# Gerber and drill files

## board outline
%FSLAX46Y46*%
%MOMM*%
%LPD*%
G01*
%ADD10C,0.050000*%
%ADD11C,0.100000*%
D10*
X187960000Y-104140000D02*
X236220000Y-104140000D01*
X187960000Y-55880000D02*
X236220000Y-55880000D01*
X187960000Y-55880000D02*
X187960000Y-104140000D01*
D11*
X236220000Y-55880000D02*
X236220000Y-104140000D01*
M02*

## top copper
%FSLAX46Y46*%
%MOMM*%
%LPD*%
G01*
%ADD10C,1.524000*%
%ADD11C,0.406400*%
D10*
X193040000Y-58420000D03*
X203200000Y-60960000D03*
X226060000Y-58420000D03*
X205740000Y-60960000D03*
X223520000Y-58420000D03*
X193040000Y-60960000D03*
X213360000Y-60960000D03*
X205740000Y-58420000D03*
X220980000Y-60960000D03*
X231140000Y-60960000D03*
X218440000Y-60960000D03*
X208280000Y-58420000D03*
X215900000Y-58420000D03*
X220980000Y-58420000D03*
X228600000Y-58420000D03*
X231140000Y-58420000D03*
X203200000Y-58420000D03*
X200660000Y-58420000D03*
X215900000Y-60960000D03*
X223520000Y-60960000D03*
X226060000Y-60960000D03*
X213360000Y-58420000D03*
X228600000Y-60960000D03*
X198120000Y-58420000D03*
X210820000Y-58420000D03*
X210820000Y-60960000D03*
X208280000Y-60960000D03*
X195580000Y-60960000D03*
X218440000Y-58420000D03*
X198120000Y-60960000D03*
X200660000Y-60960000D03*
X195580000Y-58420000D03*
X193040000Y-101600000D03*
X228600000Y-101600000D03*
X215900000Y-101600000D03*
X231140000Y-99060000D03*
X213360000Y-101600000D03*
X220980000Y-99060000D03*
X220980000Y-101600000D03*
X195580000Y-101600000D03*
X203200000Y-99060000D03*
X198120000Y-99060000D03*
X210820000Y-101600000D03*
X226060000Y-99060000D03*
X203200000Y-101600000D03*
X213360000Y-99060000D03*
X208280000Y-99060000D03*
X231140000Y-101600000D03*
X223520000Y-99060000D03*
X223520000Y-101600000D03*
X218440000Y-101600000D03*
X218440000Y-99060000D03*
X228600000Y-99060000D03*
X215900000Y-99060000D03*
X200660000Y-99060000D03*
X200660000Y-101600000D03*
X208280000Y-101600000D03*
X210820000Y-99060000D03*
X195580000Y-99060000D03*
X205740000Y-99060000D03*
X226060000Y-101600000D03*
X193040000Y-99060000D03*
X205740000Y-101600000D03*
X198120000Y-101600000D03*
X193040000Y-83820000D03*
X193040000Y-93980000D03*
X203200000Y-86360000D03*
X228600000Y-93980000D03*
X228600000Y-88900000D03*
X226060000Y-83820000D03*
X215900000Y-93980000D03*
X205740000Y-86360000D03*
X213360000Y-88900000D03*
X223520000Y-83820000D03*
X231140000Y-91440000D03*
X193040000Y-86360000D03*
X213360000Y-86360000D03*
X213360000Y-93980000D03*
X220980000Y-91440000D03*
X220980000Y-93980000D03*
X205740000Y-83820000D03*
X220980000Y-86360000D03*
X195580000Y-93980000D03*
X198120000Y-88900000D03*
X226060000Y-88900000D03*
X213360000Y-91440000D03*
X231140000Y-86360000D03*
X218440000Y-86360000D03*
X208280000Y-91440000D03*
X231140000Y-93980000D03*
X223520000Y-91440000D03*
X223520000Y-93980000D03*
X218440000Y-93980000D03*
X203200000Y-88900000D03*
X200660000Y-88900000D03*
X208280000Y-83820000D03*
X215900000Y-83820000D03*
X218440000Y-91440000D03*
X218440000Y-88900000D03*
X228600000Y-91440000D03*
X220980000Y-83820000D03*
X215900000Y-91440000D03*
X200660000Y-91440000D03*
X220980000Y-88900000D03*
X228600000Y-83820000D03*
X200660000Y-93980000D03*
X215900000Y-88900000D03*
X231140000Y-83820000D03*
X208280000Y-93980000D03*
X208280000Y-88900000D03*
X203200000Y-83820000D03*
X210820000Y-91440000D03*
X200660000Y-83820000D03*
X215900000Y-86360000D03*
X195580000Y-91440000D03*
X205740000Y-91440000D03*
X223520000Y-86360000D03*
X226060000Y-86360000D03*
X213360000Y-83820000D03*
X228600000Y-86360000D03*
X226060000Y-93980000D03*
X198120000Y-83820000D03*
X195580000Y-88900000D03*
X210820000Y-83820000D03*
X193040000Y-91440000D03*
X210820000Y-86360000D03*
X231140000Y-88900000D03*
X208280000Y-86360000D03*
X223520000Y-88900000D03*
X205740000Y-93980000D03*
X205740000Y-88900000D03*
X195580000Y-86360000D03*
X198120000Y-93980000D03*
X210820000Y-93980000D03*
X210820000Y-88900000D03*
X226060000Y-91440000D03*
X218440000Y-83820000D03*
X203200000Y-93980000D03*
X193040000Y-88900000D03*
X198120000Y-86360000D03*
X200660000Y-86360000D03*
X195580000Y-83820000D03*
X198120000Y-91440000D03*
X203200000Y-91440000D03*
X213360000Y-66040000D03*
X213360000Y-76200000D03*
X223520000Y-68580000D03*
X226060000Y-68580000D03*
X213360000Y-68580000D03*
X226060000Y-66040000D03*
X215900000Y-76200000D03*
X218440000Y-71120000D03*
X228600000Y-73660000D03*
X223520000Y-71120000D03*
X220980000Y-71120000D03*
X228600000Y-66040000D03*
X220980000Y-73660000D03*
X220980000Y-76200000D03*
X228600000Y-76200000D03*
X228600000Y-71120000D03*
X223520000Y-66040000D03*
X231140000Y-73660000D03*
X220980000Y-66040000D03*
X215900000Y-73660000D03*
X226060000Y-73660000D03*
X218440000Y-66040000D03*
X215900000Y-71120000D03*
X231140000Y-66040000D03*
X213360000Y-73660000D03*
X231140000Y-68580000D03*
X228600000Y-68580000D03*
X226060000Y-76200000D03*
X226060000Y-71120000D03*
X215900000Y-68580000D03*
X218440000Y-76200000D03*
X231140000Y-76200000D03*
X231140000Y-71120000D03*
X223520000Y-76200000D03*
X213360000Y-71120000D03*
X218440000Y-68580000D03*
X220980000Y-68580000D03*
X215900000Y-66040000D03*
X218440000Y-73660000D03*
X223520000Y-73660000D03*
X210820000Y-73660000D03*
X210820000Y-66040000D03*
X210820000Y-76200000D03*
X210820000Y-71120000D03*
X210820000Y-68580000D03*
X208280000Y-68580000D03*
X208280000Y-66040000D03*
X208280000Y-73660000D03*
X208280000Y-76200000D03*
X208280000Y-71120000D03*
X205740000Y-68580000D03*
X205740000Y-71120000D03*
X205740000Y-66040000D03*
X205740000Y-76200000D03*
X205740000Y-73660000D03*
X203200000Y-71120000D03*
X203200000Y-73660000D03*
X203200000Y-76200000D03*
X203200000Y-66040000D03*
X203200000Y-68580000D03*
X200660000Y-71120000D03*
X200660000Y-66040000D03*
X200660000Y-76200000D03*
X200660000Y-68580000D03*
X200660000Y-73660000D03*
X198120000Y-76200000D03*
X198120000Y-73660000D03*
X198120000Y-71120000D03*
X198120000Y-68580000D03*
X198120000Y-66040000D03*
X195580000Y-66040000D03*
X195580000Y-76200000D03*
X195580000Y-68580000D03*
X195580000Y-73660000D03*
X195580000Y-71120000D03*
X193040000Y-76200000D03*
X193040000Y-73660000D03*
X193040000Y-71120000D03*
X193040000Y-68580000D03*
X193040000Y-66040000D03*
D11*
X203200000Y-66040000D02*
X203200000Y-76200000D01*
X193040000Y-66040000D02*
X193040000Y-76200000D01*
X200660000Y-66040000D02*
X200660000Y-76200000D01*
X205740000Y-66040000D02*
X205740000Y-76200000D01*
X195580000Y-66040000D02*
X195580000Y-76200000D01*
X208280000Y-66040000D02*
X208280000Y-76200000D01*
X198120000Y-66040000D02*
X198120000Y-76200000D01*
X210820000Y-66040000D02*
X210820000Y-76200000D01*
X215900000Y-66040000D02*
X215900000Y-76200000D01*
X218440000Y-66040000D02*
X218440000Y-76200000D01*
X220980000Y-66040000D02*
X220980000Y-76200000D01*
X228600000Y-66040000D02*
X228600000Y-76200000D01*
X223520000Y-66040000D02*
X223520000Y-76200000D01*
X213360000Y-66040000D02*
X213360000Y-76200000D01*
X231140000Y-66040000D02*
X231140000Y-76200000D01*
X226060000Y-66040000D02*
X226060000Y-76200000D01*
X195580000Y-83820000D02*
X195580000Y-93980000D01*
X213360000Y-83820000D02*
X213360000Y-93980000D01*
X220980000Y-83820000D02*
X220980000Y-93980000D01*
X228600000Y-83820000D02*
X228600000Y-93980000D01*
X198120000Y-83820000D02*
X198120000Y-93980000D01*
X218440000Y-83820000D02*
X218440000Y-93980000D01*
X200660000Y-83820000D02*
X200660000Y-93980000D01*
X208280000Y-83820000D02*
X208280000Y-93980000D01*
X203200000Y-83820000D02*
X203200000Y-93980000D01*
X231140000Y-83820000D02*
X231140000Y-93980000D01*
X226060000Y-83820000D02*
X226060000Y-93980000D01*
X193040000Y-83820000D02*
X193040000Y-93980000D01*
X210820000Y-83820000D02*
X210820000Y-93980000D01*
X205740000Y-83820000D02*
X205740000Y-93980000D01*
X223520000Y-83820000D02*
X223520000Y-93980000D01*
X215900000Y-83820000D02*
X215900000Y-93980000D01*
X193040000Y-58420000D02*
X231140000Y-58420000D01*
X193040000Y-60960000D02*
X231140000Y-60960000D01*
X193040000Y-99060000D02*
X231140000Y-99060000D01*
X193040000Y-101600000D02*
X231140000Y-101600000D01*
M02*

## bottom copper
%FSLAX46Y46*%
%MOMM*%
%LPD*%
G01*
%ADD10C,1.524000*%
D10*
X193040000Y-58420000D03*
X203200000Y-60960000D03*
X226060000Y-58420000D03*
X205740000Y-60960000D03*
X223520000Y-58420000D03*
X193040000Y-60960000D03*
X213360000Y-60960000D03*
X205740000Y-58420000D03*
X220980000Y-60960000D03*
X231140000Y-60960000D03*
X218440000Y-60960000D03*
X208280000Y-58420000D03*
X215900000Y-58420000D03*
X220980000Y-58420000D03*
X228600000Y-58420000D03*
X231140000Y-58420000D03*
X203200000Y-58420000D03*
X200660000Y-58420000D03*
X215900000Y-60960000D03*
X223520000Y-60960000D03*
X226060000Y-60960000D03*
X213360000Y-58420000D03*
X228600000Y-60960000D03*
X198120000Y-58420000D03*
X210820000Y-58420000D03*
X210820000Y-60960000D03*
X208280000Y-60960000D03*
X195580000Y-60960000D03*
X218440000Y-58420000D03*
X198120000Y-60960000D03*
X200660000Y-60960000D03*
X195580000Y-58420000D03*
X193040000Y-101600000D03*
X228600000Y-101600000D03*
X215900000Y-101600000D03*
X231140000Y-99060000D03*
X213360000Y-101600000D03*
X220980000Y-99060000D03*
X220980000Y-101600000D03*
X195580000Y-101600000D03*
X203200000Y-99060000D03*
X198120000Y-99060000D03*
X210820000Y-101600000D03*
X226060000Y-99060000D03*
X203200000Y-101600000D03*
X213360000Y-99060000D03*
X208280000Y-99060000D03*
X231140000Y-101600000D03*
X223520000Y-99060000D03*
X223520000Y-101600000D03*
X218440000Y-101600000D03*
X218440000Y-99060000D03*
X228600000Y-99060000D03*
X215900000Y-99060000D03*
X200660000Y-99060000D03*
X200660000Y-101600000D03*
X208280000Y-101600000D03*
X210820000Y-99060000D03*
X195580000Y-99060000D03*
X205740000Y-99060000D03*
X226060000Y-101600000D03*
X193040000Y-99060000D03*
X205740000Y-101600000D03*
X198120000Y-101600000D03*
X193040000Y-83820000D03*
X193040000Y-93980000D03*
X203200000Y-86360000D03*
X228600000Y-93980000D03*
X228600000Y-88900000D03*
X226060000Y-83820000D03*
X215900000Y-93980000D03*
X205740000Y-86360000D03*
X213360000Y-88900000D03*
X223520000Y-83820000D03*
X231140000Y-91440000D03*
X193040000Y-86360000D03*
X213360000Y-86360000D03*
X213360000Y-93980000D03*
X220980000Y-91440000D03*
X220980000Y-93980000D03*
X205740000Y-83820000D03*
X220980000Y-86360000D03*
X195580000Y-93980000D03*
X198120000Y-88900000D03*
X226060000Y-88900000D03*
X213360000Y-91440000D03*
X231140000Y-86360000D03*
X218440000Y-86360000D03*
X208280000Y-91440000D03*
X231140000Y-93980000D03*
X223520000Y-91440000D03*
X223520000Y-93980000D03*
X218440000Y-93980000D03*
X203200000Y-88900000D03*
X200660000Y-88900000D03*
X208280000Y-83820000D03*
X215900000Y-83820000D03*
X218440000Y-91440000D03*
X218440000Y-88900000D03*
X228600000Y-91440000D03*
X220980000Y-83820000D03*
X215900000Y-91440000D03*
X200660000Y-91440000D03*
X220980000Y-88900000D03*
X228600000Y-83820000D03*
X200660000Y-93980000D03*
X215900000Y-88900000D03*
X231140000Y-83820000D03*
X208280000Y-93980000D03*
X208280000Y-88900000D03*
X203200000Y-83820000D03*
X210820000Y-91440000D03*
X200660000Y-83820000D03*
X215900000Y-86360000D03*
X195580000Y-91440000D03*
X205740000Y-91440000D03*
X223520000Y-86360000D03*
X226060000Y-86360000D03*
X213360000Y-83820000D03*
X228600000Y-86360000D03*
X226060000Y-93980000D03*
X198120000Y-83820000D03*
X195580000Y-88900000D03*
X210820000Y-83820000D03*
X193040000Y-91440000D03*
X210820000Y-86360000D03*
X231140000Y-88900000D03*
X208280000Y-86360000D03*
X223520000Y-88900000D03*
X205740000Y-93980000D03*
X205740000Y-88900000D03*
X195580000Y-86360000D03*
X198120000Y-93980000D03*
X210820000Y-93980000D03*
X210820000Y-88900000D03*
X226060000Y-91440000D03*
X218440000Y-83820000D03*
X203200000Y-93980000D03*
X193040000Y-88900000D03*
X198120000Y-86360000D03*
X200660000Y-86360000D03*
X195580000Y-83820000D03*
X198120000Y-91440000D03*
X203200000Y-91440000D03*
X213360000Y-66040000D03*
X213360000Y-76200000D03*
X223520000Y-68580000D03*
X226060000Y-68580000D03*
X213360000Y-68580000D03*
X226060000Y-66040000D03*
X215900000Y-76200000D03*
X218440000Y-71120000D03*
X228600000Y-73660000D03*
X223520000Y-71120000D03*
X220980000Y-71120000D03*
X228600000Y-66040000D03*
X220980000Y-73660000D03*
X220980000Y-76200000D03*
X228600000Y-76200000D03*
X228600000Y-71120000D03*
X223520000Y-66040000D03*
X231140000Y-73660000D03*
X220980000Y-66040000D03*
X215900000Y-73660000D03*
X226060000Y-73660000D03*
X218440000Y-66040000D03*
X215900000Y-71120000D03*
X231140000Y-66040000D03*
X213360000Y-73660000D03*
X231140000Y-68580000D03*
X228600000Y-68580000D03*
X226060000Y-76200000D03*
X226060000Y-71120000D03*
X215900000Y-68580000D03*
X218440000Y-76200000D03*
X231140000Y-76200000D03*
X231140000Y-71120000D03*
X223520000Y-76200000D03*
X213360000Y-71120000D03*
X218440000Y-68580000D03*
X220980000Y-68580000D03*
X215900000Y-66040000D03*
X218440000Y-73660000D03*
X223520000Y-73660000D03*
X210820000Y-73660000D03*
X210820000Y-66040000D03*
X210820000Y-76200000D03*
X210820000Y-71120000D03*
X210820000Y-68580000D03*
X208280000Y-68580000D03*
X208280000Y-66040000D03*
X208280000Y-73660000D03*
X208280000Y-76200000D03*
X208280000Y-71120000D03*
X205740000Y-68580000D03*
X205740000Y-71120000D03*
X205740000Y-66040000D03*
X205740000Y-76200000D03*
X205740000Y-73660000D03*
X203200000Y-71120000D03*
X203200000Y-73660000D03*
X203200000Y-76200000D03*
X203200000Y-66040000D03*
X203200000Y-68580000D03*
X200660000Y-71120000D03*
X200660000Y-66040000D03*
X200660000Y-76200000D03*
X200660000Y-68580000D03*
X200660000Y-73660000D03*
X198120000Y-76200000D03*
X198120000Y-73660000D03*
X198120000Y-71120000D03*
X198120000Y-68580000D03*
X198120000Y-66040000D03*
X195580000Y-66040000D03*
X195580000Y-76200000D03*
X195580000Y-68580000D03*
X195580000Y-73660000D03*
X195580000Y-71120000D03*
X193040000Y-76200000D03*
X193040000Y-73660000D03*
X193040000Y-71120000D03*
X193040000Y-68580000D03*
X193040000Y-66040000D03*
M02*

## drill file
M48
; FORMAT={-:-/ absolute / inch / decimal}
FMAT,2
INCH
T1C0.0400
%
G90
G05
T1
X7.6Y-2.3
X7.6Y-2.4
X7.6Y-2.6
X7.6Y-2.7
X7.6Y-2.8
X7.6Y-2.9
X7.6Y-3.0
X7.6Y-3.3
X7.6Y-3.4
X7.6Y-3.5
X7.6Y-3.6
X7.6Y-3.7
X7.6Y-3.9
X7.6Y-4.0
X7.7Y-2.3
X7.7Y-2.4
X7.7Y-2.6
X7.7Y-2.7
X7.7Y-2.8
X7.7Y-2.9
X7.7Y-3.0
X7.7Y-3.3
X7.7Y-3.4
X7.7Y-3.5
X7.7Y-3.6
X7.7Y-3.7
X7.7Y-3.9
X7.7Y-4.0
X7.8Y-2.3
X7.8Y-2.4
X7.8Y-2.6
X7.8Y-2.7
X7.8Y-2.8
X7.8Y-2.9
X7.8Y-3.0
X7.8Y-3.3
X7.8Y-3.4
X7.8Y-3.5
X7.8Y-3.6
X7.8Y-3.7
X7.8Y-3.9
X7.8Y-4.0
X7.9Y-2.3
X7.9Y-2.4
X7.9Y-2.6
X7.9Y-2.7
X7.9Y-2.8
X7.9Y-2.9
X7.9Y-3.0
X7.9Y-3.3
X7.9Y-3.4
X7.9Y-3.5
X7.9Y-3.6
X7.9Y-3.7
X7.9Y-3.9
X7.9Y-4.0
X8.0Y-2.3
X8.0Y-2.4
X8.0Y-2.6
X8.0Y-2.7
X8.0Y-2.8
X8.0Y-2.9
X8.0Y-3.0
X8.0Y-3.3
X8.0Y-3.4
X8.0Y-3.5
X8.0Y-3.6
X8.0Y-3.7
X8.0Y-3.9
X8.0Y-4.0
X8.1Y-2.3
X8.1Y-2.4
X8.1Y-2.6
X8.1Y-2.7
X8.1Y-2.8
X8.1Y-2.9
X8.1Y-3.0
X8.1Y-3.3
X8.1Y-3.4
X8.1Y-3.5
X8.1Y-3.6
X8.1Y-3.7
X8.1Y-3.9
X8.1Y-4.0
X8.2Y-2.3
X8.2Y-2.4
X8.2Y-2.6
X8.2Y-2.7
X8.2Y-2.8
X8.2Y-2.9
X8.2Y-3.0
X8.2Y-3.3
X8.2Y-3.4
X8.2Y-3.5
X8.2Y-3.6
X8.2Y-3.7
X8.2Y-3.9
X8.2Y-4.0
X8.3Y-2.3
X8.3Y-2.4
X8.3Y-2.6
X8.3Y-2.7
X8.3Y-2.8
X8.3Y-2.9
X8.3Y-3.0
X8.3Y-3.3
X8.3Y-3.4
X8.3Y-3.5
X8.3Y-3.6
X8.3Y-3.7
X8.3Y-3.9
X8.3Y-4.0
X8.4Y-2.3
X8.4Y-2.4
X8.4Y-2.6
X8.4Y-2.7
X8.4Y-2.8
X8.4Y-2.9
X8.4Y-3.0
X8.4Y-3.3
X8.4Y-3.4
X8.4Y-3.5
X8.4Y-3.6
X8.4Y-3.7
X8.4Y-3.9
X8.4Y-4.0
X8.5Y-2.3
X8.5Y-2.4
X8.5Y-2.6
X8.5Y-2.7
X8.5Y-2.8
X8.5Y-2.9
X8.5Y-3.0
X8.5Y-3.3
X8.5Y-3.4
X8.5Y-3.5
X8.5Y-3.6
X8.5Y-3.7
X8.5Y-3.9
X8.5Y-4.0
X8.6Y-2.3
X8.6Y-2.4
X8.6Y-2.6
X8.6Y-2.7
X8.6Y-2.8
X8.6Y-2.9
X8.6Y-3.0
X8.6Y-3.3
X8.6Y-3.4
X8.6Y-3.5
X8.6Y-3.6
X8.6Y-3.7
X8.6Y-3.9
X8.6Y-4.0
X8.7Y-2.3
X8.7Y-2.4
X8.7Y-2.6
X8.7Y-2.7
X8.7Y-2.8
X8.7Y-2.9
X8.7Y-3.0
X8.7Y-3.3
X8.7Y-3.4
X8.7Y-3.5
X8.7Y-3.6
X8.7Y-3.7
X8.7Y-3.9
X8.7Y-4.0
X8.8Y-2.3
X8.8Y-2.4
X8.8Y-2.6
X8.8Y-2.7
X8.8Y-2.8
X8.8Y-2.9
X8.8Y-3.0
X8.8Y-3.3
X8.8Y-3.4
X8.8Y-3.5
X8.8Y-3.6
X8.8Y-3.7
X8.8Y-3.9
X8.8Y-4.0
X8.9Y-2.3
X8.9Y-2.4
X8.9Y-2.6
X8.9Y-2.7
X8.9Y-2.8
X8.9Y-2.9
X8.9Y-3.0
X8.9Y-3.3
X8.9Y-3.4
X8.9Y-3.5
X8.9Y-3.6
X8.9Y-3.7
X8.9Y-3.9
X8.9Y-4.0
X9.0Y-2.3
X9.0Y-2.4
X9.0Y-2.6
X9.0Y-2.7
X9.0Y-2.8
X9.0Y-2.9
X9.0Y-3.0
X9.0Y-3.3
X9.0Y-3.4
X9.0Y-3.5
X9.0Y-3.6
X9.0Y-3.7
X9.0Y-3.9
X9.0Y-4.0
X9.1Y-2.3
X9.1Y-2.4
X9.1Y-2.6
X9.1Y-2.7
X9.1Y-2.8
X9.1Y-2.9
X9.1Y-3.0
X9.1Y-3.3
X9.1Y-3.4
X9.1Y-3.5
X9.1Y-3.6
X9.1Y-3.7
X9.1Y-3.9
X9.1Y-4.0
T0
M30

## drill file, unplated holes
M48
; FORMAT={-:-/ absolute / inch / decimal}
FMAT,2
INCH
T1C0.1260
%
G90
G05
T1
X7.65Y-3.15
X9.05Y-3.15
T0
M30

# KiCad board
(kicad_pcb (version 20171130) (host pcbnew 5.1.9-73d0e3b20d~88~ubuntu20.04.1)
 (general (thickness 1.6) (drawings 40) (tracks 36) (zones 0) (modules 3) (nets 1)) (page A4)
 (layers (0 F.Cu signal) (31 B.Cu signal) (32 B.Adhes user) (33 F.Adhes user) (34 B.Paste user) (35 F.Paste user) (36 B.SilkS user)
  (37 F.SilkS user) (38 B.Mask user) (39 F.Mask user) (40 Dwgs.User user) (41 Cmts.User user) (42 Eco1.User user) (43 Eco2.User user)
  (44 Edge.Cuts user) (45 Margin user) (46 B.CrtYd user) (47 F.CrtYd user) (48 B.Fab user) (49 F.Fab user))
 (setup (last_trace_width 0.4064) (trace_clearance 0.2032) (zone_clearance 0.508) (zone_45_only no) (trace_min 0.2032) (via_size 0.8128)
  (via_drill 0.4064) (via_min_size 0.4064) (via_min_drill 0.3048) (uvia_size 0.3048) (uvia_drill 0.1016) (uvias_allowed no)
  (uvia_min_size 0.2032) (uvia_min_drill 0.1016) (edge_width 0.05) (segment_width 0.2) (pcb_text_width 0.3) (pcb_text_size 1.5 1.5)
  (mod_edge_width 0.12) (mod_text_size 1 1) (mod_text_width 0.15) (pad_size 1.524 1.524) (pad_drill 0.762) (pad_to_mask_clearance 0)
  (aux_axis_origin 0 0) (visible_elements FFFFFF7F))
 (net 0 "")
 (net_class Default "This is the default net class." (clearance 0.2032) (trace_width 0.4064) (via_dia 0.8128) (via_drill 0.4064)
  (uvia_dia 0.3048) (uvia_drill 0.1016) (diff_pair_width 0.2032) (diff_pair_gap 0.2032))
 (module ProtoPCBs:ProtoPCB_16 (layer F.Cu) (at 193.04 58.42)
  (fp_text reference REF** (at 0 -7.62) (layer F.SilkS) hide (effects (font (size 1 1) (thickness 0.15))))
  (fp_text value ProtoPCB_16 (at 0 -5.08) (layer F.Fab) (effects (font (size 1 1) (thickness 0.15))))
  (pad 1 thru_hole circle (at 0 0) (size 1.524 1.524) (drill 1.016) (layers *.Cu *.Mask))
  (pad 1 thru_hole circle (at 10.16 2.54) (size 1.524 1.524) (drill 1.016) (layers *.Cu *.Mask))
  (pad 1 thru_hole circle (at 33.02 0) (size 1.524 1.524) (drill 1.016) (layers *.Cu *.Mask))
  (pad 1 thru_hole circle (at 12.7 2.54) (size 1.524 1.524) (drill 1.016) (layers *.Cu *.Mask))
  (pad 1 thru_hole circle (at 30.48 0) (size 1.524 1.524) (drill 1.016) (layers *.Cu *.Mask))
  (pad 1 thru_hole circle (at 0 2.54) (size 1.524 1.524) (drill 1.016) (layers *.Cu *.Mask))
  (pad 1 thru_hole circle (at 20.32 2.54) (size 1.524 1.524) (drill 1.016) (layers *.Cu *.Mask))
  (pad 1 thru_hole circle (at 12.7 0) (size 1.524 1.524) (drill 1.016) (layers *.Cu *.Mask))
  (pad 1 thru_hole circle (at 27.94 2.54) (size 1.524 1.524) (drill 1.016) (layers *.Cu *.Mask))
  (pad 1 thru_hole circle (at 38.1 2.54) (size 1.524 1.524) (drill 1.016) (layers *.Cu *.Mask))
  (pad 1 thru_hole circle (at 25.4 2.54) (size 1.524 1.524) (drill 1.016) (layers *.Cu *.Mask))
  (pad 1 thru_hole circle (at 15.24 0) (size 1.524 1.524) (drill 1.016) (layers *.Cu *.Mask))
  (pad 1 thru_hole circle (at 22.86 0) (size 1.524 1.524) (drill 1.016) (layers *.Cu *.Mask))
  (pad 1 thru_hole circle (at 27.94 0) (size 1.524 1.524) (drill 1.016) (layers *.Cu *.Mask))
  (pad 1 thru_hole circle (at 35.56 0) (size 1.524 1.524) (drill 1.016) (layers *.Cu *.Mask))
  (pad 1 thru_hole circle (at 38.1 0) (size 1.524 1.524) (drill 1.016) (layers *.Cu *.Mask))
  (pad 1 thru_hole circle (at 10.16 0) (size 1.524 1.524) (drill 1.016) (layers *.Cu *.Mask))
  (pad 1 thru_hole circle (at 7.62 0) (size 1.524 1.524) (drill 1.016) (layers *.Cu *.Mask))
  (pad 1 thru_hole circle (at 22.86 2.54) (size 1.524 1.524) (drill 1.016) (layers *.Cu *.Mask))
  (pad 1 thru_hole circle (at 30.48 2.54) (size 1.524 1.524) (drill 1.016) (layers *.Cu *.Mask))
  (pad 1 thru_hole circle (at 33.02 2.54) (size 1.524 1.524) (drill 1.016) (layers *.Cu *.Mask))
  (pad 1 thru_hole circle (at 20.32 0) (size 1.524 1.524) (drill 1.016) (layers *.Cu *.Mask))
  (pad 1 thru_hole circle (at 35.56 2.54) (size 1.524 1.524) (drill 1.016) (layers *.Cu *.Mask))
  (pad 1 thru_hole circle (at 5.08 0) (size 1.524 1.524) (drill 1.016) (layers *.Cu *.Mask))
  (pad 1 thru_hole circle (at 17.78 0) (size 1.524 1.524) (drill 1.016) (layers *.Cu *.Mask))
  (pad 1 thru_hole circle (at 17.78 2.54) (size 1.524 1.524) (drill 1.016) (layers *.Cu *.Mask))
  (pad 1 thru_hole circle (at 15.24 2.54) (size 1.524 1.524) (drill 1.016) (layers *.Cu *.Mask))
  (pad 1 thru_hole circle (at 2.54 2.54) (size 1.524 1.524) (drill 1.016) (layers *.Cu *.Mask))
  (pad 1 thru_hole circle (at 25.4 0) (size 1.524 1.524) (drill 1.016) (layers *.Cu *.Mask))
  (pad 1 thru_hole circle (at 5.08 2.54) (size 1.524 1.524) (drill 1.016) (layers *.Cu *.Mask))
  (pad 1 thru_hole circle (at 7.62 2.54) (size 1.524 1.524) (drill 1.016) (layers *.Cu *.Mask))
  (pad 1 thru_hole circle (at 2.54 0) (size 1.524 1.524) (drill 1.016) (layers *.Cu *.Mask))
  (pad 1 thru_hole circle (at 0 43.18) (size 1.524 1.524) (drill 1.016) (layers *.Cu *.Mask))
  (pad 1 thru_hole circle (at 35.56 43.18) (size 1.524 1.524) (drill 1.016) (layers *.Cu *.Mask))
  (pad 1 thru_hole circle (at 22.86 43.18) (size 1.524 1.524) (drill 1.016) (layers *.Cu *.Mask))
  (pad 1 thru_hole circle (at 38.1 40.64) (size 1.524 1.524) (drill 1.016) (layers *.Cu *.Mask))
  (pad 1 thru_hole circle (at 20.32 43.18) (size 1.524 1.524) (drill 1.016) (layers *.Cu *.Mask))
  (pad 1 thru_hole circle (at 27.94 40.64) (size 1.524 1.524) (drill 1.016) (layers *.Cu *.Mask))
  (pad 1 thru_hole circle (at 27.94 43.18) (size 1.524 1.524) (drill 1.016) (layers *.Cu *.Mask))
  (pad 1 thru_hole circle (at 2.54 43.18) (size 1.524 1.524) (drill 1.016) (layers *.Cu *.Mask))
  (pad 1 thru_hole circle (at 10.16 40.64) (size 1.524 1.524) (drill 1.016) (layers *.Cu *.Mask))
  (pad 1 thru_hole circle (at 5.08 40.64) (size 1.524 1.524) (drill 1.016) (layers *.Cu *.Mask))
  (pad 1 thru_hole circle (at 17.78 43.18) (size 1.524 1.524) (drill 1.016) (layers *.Cu *.Mask))
  (pad 1 thru_hole circle (at 33.02 40.64) (size 1.524 1.524) (drill 1.016) (layers *.Cu *.Mask))
  (pad 1 thru_hole circle (at 10.16 43.18) (size 1.524 1.524) (drill 1.016) (layers *.Cu *.Mask))
  (pad 1 thru_hole circle (at 20.32 40.64) (size 1.524 1.524) (drill 1.016) (layers *.Cu *.Mask))
  (pad 1 thru_hole circle (at 15.24 40.64) (size 1.524 1.524) (drill 1.016) (layers *.Cu *.Mask))
  (pad 1 thru_hole circle (at 38.1 43.18) (size 1.524 1.524) (drill 1.016) (layers *.Cu *.Mask))
  (pad 1 thru_hole circle (at 30.48 40.64) (size 1.524 1.524) (drill 1.016) (layers *.Cu *.Mask))
  (pad 1 thru_hole circle (at 30.48 43.18) (size 1.524 1.524) (drill 1.016) (layers *.Cu *.Mask))
  (pad 1 thru_hole circle (at 25.4 43.18) (size 1.524 1.524) (drill 1.016) (layers *.Cu *.Mask))
  (pad 1 thru_hole circle (at 25.4 40.64) (size 1.524 1.524) (drill 1.016) (layers *.Cu *.Mask))
  (pad 1 thru_hole circle (at 35.56 40.64) (size 1.524 1.524) (drill 1.016) (layers *.Cu *.Mask))
  (pad 1 thru_hole circle (at 22.86 40.64) (size 1.524 1.524) (drill 1.016) (layers *.Cu *.Mask))
  (pad 1 thru_hole circle (at 7.62 40.64) (size 1.524 1.524) (drill 1.016) (layers *.Cu *.Mask))
  (pad 1 thru_hole circle (at 7.62 43.18) (size 1.524 1.524) (drill 1.016) (layers *.Cu *.Mask))
  (pad 1 thru_hole circle (at 15.24 43.18) (size 1.524 1.524) (drill 1.016) (layers *.Cu *.Mask))
  (pad 1 thru_hole circle (at 17.78 40.64) (size 1.524 1.524) (drill 1.016) (layers *.Cu *.Mask))
  (pad 1 thru_hole circle (at 2.54 40.64) (size 1.524 1.524) (drill 1.016) (layers *.Cu *.Mask))
  (pad 1 thru_hole circle (at 12.7 40.64) (size 1.524 1.524) (drill 1.016) (layers *.Cu *.Mask))
  (pad 1 thru_hole circle (at 33.02 43.18) (size 1.524 1.524) (drill 1.016) (layers *.Cu *.Mask))
  (pad 1 thru_hole circle (at 0 40.64) (size 1.524 1.524) (drill 1.016) (layers *.Cu *.Mask))
  (pad 1 thru_hole circle (at 12.7 43.18) (size 1.524 1.524) (drill 1.016) (layers *.Cu *.Mask))
  (pad 1 thru_hole circle (at 5.08 43.18) (size 1.524 1.524) (drill 1.016) (layers *.Cu *.Mask))
  (pad 1 thru_hole circle (at 0 25.4) (size 1.524 1.524) (drill 1.016) (layers *.Cu *.Mask))
  (pad 1 thru_hole circle (at 0 35.56) (size 1.524 1.524) (drill 1.016) (layers *.Cu *.Mask))
  (pad 1 thru_hole circle (at 10.16 27.94) (size 1.524 1.524) (drill 1.016) (layers *.Cu *.Mask))
  (pad 1 thru_hole circle (at 35.56 35.56) (size 1.524 1.524) (drill 1.016) (layers *.Cu *.Mask))
  (pad 1 thru_hole circle (at 35.56 30.48) (size 1.524 1.524) (drill 1.016) (layers *.Cu *.Mask))
  (pad 1 thru_hole circle (at 33.02 25.4) (size 1.524 1.524) (drill 1.016) (layers *.Cu *.Mask))
  (pad 1 thru_hole circle (at 22.86 35.56) (size 1.524 1.524) (drill 1.016) (layers *.Cu *.Mask))
  (pad 1 thru_hole circle (at 12.7 27.94) (size 1.524 1.524) (drill 1.016) (layers *.Cu *.Mask))
  (pad 1 thru_hole circle (at 20.32 30.48) (size 1.524 1.524) (drill 1.016) (layers *.Cu *.Mask))
  (pad 1 thru_hole circle (at 30.48 25.4) (size 1.524 1.524) (drill 1.016) (layers *.Cu *.Mask))
  (pad 1 thru_hole circle (at 38.1 33.02) (size 1.524 1.524) (drill 1.016) (layers *.Cu *.Mask))
  (pad 1 thru_hole circle (at 0 27.94) (size 1.524 1.524) (drill 1.016) (layers *.Cu *.Mask))
  (pad 1 thru_hole circle (at 20.32 27.94) (size 1.524 1.524) (drill 1.016) (layers *.Cu *.Mask))
  (pad 1 thru_hole circle (at 20.32 35.56) (size 1.524 1.524) (drill 1.016) (layers *.Cu *.Mask))
  (pad 1 thru_hole circle (at 27.94 33.02) (size 1.524 1.524) (drill 1.016) (layers *.Cu *.Mask))
  (pad 1 thru_hole circle (at 27.94 35.56) (size 1.524 1.524) (drill 1.016) (layers *.Cu *.Mask))
  (pad 1 thru_hole circle (at 12.7 25.4) (size 1.524 1.524) (drill 1.016) (layers *.Cu *.Mask))
  (pad 1 thru_hole circle (at 27.94 27.94) (size 1.524 1.524) (drill 1.016) (layers *.Cu *.Mask))
  (pad 1 thru_hole circle (at 2.54 35.56) (size 1.524 1.524) (drill 1.016) (layers *.Cu *.Mask))
  (pad 1 thru_hole circle (at 5.08 30.48) (size 1.524 1.524) (drill 1.016) (layers *.Cu *.Mask))
  (pad 1 thru_hole circle (at 33.02 30.48) (size 1.524 1.524) (drill 1.016) (layers *.Cu *.Mask))
  (pad 1 thru_hole circle (at 20.32 33.02) (size 1.524 1.524) (drill 1.016) (layers *.Cu *.Mask))
  (pad 1 thru_hole circle (at 38.1 27.94) (size 1.524 1.524) (drill 1.016) (layers *.Cu *.Mask))
  (pad 1 thru_hole circle (at 25.4 27.94) (size 1.524 1.524) (drill 1.016) (layers *.Cu *.Mask))
  (pad 1 thru_hole circle (at 15.24 33.02) (size 1.524 1.524) (drill 1.016) (layers *.Cu *.Mask))
  (pad 1 thru_hole circle (at 38.1 35.56) (size 1.524 1.524) (drill 1.016) (layers *.Cu *.Mask))
  (pad 1 thru_hole circle (at 30.48 33.02) (size 1.524 1.524) (drill 1.016) (layers *.Cu *.Mask))
  (pad 1 thru_hole circle (at 30.48 35.56) (size 1.524 1.524) (drill 1.016) (layers *.Cu *.Mask))
  (pad 1 thru_hole circle (at 25.4 35.56) (size 1.524 1.524) (drill 1.016) (layers *.Cu *.Mask))
  (pad 1 thru_hole circle (at 10.16 30.48) (size 1.524 1.524) (drill 1.016) (layers *.Cu *.Mask))
  (pad 1 thru_hole circle (at 7.62 30.48) (size 1.524 1.524) (drill 1.016) (layers *.Cu *.Mask))
  (pad 1 thru_hole circle (at 15.24 25.4) (size 1.524 1.524) (drill 1.016) (layers *.Cu *.Mask))
  (pad 1 thru_hole circle (at 22.86 25.4) (size 1.524 1.524) (drill 1.016) (layers *.Cu *.Mask))
  (pad 1 thru_hole circle (at 25.4 33.02) (size 1.524 1.524) (drill 1.016) (layers *.Cu *.Mask))
  (pad 1 thru_hole circle (at 25.4 30.48) (size 1.524 1.524) (drill 1.016) (layers *.Cu *.Mask))
  (pad 1 thru_hole circle (at 35.56 33.02) (size 1.524 1.524) (drill 1.016) (layers *.Cu *.Mask))
  (pad 1 thru_hole circle (at 27.94 25.4) (size 1.524 1.524) (drill 1.016) (layers *.Cu *.Mask))
  (pad 1 thru_hole circle (at 22.86 33.02) (size 1.524 1.524) (drill 1.016) (layers *.Cu *.Mask))
  (pad 1 thru_hole circle (at 7.62 33.02) (size 1.524 1.524) (drill 1.016) (layers *.Cu *.Mask))
  (pad 1 thru_hole circle (at 27.94 30.48) (size 1.524 1.524) (drill 1.016) (layers *.Cu *.Mask))
  (pad 1 thru_hole circle (at 35.56 25.4) (size 1.524 1.524) (drill 1.016) (layers *.Cu *.Mask))
  (pad 1 thru_hole circle (at 7.62 35.56) (size 1.524 1.524) (drill 1.016) (layers *.Cu *.Mask))
  (pad 1 thru_hole circle (at 22.86 30.48) (size 1.524 1.524) (drill 1.016) (layers *.Cu *.Mask))
  (pad 1 thru_hole circle (at 38.1 25.4) (size 1.524 1.524) (drill 1.016) (layers *.Cu *.Mask))
  (pad 1 thru_hole circle (at 15.24 35.56) (size 1.524 1.524) (drill 1.016) (layers *.Cu *.Mask))
  (pad 1 thru_hole circle (at 15.24 30.48) (size 1.524 1.524) (drill 1.016) (layers *.Cu *.Mask))
  (pad 1 thru_hole circle (at 10.16 25.4) (size 1.524 1.524) (drill 1.016) (layers *.Cu *.Mask))
  (pad 1 thru_hole circle (at 17.78 33.02) (size 1.524 1.524) (drill 1.016) (layers *.Cu *.Mask))
  (pad 1 thru_hole circle (at 7.62 25.4) (size 1.524 1.524) (drill 1.016) (layers *.Cu *.Mask))
  (pad 1 thru_hole circle (at 22.86 27.94) (size 1.524 1.524) (drill 1.016) (layers *.Cu *.Mask))
  (pad 1 thru_hole circle (at 2.54 33.02) (size 1.524 1.524) (drill 1.016) (layers *.Cu *.Mask))
  (pad 1 thru_hole circle (at 12.7 33.02) (size 1.524 1.524) (drill 1.016) (layers *.Cu *.Mask))
  (pad 1 thru_hole circle (at 30.48 27.94) (size 1.524 1.524) (drill 1.016) (layers *.Cu *.Mask))
  (pad 1 thru_hole circle (at 33.02 27.94) (size 1.524 1.524) (drill 1.016) (layers *.Cu *.Mask))
  (pad 1 thru_hole circle (at 20.32 25.4) (size 1.524 1.524) (drill 1.016) (layers *.Cu *.Mask))
  (pad 1 thru_hole circle (at 35.56 27.94) (size 1.524 1.524) (drill 1.016) (layers *.Cu *.Mask))
  (pad 1 thru_hole circle (at 33.02 35.56) (size 1.524 1.524) (drill 1.016) (layers *.Cu *.Mask))
  (pad 1 thru_hole circle (at 5.08 25.4) (size 1.524 1.524) (drill 1.016) (layers *.Cu *.Mask))
  (pad 1 thru_hole circle (at 2.54 30.48) (size 1.524 1.524) (drill 1.016) (layers *.Cu *.Mask))
  (pad 1 thru_hole circle (at 17.78 25.4) (size 1.524 1.524) (drill 1.016) (layers *.Cu *.Mask))
  (pad 1 thru_hole circle (at 0 33.02) (size 1.524 1.524) (drill 1.016) (layers *.Cu *.Mask))
  (pad 1 thru_hole circle (at 17.78 27.94) (size 1.524 1.524) (drill 1.016) (layers *.Cu *.Mask))
  (pad 1 thru_hole circle (at 38.1 30.48) (size 1.524 1.524) (drill 1.016) (layers *.Cu *.Mask))
  (pad 1 thru_hole circle (at 15.24 27.94) (size 1.524 1.524) (drill 1.016) (layers *.Cu *.Mask))
  (pad 1 thru_hole circle (at 30.48 30.48) (size 1.524 1.524) (drill 1.016) (layers *.Cu *.Mask))
  (pad 1 thru_hole circle (at 12.7 35.56) (size 1.524 1.524) (drill 1.016) (layers *.Cu *.Mask))
  (pad 1 thru_hole circle (at 12.7 30.48) (size 1.524 1.524) (drill 1.016) (layers *.Cu *.Mask))
  (pad 1 thru_hole circle (at 2.54 27.94) (size 1.524 1.524) (drill 1.016) (layers *.Cu *.Mask))
  (pad 1 thru_hole circle (at 5.08 35.56) (size 1.524 1.524) (drill 1.016) (layers *.Cu *.Mask))
  (pad 1 thru_hole circle (at 17.78 35.56) (size 1.524 1.524) (drill 1.016) (layers *.Cu *.Mask))
  (pad 1 thru_hole circle (at 17.78 30.48) (size 1.524 1.524) (drill 1.016) (layers *.Cu *.Mask))
  (pad 1 thru_hole circle (at 33.02 33.02) (size 1.524 1.524) (drill 1.016) (layers *.Cu *.Mask))
  (pad 1 thru_hole circle (at 25.4 25.4) (size 1.524 1.524) (drill 1.016) (layers *.Cu *.Mask))
  (pad 1 thru_hole circle (at 10.16 35.56) (size 1.524 1.524) (drill 1.016) (layers *.Cu *.Mask))
  (pad 1 thru_hole circle (at 0 30.48) (size 1.524 1.524) (drill 1.016) (layers *.Cu *.Mask))
  (pad 1 thru_hole circle (at 5.08 27.94) (size 1.524 1.524) (drill 1.016) (layers *.Cu *.Mask))
  (pad 1 thru_hole circle (at 7.62 27.94) (size 1.524 1.524) (drill 1.016) (layers *.Cu *.Mask))
  (pad 1 thru_hole circle (at 2.54 25.4) (size 1.524 1.524) (drill 1.016) (layers *.Cu *.Mask))
  (pad 1 thru_hole circle (at 5.08 33.02) (size 1.524 1.524) (drill 1.016) (layers *.Cu *.Mask))
  (pad 1 thru_hole circle (at 10.16 33.02) (size 1.524 1.524) (drill 1.016) (layers *.Cu *.Mask))
  (pad 1 thru_hole circle (at 20.32 7.62) (size 1.524 1.524) (drill 1.016) (layers *.Cu *.Mask))
  (pad 1 thru_hole circle (at 20.32 17.78) (size 1.524 1.524) (drill 1.016) (layers *.Cu *.Mask))
  (pad 1 thru_hole circle (at 30.48 10.16) (size 1.524 1.524) (drill 1.016) (layers *.Cu *.Mask))
  (pad 1 thru_hole circle (at 33.02 10.16) (size 1.524 1.524) (drill 1.016) (layers *.Cu *.Mask))
  (pad 1 thru_hole circle (at 20.32 10.16) (size 1.524 1.524) (drill 1.016) (layers *.Cu *.Mask))
  (pad 1 thru_hole circle (at 33.02 7.62) (size 1.524 1.524) (drill 1.016) (layers *.Cu *.Mask))
  (pad 1 thru_hole circle (at 22.86 17.78) (size 1.524 1.524) (drill 1.016) (layers *.Cu *.Mask))
  (pad 1 thru_hole circle (at 25.4 12.7) (size 1.524 1.524) (drill 1.016) (layers *.Cu *.Mask))
  (pad 1 thru_hole circle (at 35.56 15.24) (size 1.524 1.524) (drill 1.016) (layers *.Cu *.Mask))
  (pad 1 thru_hole circle (at 30.48 12.7) (size 1.524 1.524) (drill 1.016) (layers *.Cu *.Mask))
  (pad 1 thru_hole circle (at 27.94 12.7) (size 1.524 1.524) (drill 1.016) (layers *.Cu *.Mask))
  (pad 1 thru_hole circle (at 35.56 7.62) (size 1.524 1.524) (drill 1.016) (layers *.Cu *.Mask))
  (pad 1 thru_hole circle (at 27.94 15.24) (size 1.524 1.524) (drill 1.016) (layers *.Cu *.Mask))
  (pad 1 thru_hole circle (at 27.94 17.78) (size 1.524 1.524) (drill 1.016) (layers *.Cu *.Mask))
  (pad 1 thru_hole circle (at 35.56 17.78) (size 1.524 1.524) (drill 1.016) (layers *.Cu *.Mask))
  (pad 1 thru_hole circle (at 35.56 12.7) (size 1.524 1.524) (drill 1.016) (layers *.Cu *.Mask))
  (pad 1 thru_hole circle (at 30.48 7.62) (size 1.524 1.524) (drill 1.016) (layers *.Cu *.Mask))
  (pad 1 thru_hole circle (at 38.1 15.24) (size 1.524 1.524) (drill 1.016) (layers *.Cu *.Mask))
  (pad 1 thru_hole circle (at 27.94 7.62) (size 1.524 1.524) (drill 1.016) (layers *.Cu *.Mask))
  (pad 1 thru_hole circle (at 22.86 15.24) (size 1.524 1.524) (drill 1.016) (layers *.Cu *.Mask))
  (pad 1 thru_hole circle (at 33.02 15.24) (size 1.524 1.524) (drill 1.016) (layers *.Cu *.Mask))
  (pad 1 thru_hole circle (at 25.4 7.62) (size 1.524 1.524) (drill 1.016) (layers *.Cu *.Mask))
  (pad 1 thru_hole circle (at 22.86 12.7) (size 1.524 1.524) (drill 1.016) (layers *.Cu *.Mask))
  (pad 1 thru_hole circle (at 38.1 7.62) (size 1.524 1.524) (drill 1.016) (layers *.Cu *.Mask))
  (pad 1 thru_hole circle (at 20.32 15.24) (size 1.524 1.524) (drill 1.016) (layers *.Cu *.Mask))
  (pad 1 thru_hole circle (at 38.1 10.16) (size 1.524 1.524) (drill 1.016) (layers *.Cu *.Mask))
  (pad 1 thru_hole circle (at 35.56 10.16) (size 1.524 1.524) (drill 1.016) (layers *.Cu *.Mask))
  (pad 1 thru_hole circle (at 33.02 17.78) (size 1.524 1.524) (drill 1.016) (layers *.Cu *.Mask))
  (pad 1 thru_hole circle (at 33.02 12.7) (size 1.524 1.524) (drill 1.016) (layers *.Cu *.Mask))
  (pad 1 thru_hole circle (at 22.86 10.16) (size 1.524 1.524) (drill 1.016) (layers *.Cu *.Mask))
  (pad 1 thru_hole circle (at 25.4 17.78) (size 1.524 1.524) (drill 1.016) (layers *.Cu *.Mask))
  (pad 1 thru_hole circle (at 38.1 17.78) (size 1.524 1.524) (drill 1.016) (layers *.Cu *.Mask))
  (pad 1 thru_hole circle (at 38.1 12.7) (size 1.524 1.524) (drill 1.016) (layers *.Cu *.Mask))
  (pad 1 thru_hole circle (at 30.48 17.78) (size 1.524 1.524) (drill 1.016) (layers *.Cu *.Mask))
  (pad 1 thru_hole circle (at 20.32 12.7) (size 1.524 1.524) (drill 1.016) (layers *.Cu *.Mask))
  (pad 1 thru_hole circle (at 25.4 10.16) (size 1.524 1.524) (drill 1.016) (layers *.Cu *.Mask))
  (pad 1 thru_hole circle (at 27.94 10.16) (size 1.524 1.524) (drill 1.016) (layers *.Cu *.Mask))
  (pad 1 thru_hole circle (at 22.86 7.62) (size 1.524 1.524) (drill 1.016) (layers *.Cu *.Mask))
  (pad 1 thru_hole circle (at 25.4 15.24) (size 1.524 1.524) (drill 1.016) (layers *.Cu *.Mask))
  (pad 1 thru_hole circle (at 30.48 15.24) (size 1.524 1.524) (drill 1.016) (layers *.Cu *.Mask))
  (pad 1 thru_hole circle (at 17.78 15.24) (size 1.524 1.524) (drill 1.016) (layers *.Cu *.Mask))
  (pad 1 thru_hole circle (at 17.78 7.62) (size 1.524 1.524) (drill 1.016) (layers *.Cu *.Mask))
  (pad 1 thru_hole circle (at 17.78 17.78) (size 1.524 1.524) (drill 1.016) (layers *.Cu *.Mask))
  (pad 1 thru_hole circle (at 17.78 12.7) (size 1.524 1.524) (drill 1.016) (layers *.Cu *.Mask))
  (pad 1 thru_hole circle (at 17.78 10.16) (size 1.524 1.524) (drill 1.016) (layers *.Cu *.Mask))
  (pad 1 thru_hole circle (at 15.24 10.16) (size 1.524 1.524) (drill 1.016) (layers *.Cu *.Mask))
  (pad 1 thru_hole circle (at 15.24 7.62) (size 1.524 1.524) (drill 1.016) (layers *.Cu *.Mask))
  (pad 1 thru_hole circle (at 15.24 15.24) (size 1.524 1.524) (drill 1.016) (layers *.Cu *.Mask))
  (pad 1 thru_hole circle (at 15.24 17.78) (size 1.524 1.524) (drill 1.016) (layers *.Cu *.Mask))
  (pad 1 thru_hole circle (at 15.24 12.7) (size 1.524 1.524) (drill 1.016) (layers *.Cu *.Mask))
  (pad 1 thru_hole circle (at 12.7 10.16) (size 1.524 1.524) (drill 1.016) (layers *.Cu *.Mask))
  (pad 1 thru_hole circle (at 12.7 12.7) (size 1.524 1.524) (drill 1.016) (layers *.Cu *.Mask))
  (pad 1 thru_hole circle (at 12.7 7.62) (size 1.524 1.524) (drill 1.016) (layers *.Cu *.Mask))
  (pad 1 thru_hole circle (at 12.7 17.78) (size 1.524 1.524) (drill 1.016) (layers *.Cu *.Mask))
  (pad 1 thru_hole circle (at 12.7 15.24) (size 1.524 1.524) (drill 1.016) (layers *.Cu *.Mask))
  (pad 1 thru_hole circle (at 10.16 12.7) (size 1.524 1.524) (drill 1.016) (layers *.Cu *.Mask))
  (pad 1 thru_hole circle (at 10.16 15.24) (size 1.524 1.524) (drill 1.016) (layers *.Cu *.Mask))
  (pad 1 thru_hole circle (at 10.16 17.78) (size 1.524 1.524) (drill 1.016) (layers *.Cu *.Mask))
  (pad 1 thru_hole circle (at 10.16 7.62) (size 1.524 1.524) (drill 1.016) (layers *.Cu *.Mask))
  (pad 1 thru_hole circle (at 10.16 10.16) (size 1.524 1.524) (drill 1.016) (layers *.Cu *.Mask))
  (pad 1 thru_hole circle (at 7.62 12.7) (size 1.524 1.524) (drill 1.016) (layers *.Cu *.Mask))
  (pad 1 thru_hole circle (at 7.62 7.62) (size 1.524 1.524) (drill 1.016) (layers *.Cu *.Mask))
  (pad 1 thru_hole circle (at 7.62 17.78) (size 1.524 1.524) (drill 1.016) (layers *.Cu *.Mask))
  (pad 1 thru_hole circle (at 7.62 10.16) (size 1.524 1.524) (drill 1.016) (layers *.Cu *.Mask))
  (pad 1 thru_hole circle (at 7.62 15.24) (size 1.524 1.524) (drill 1.016) (layers *.Cu *.Mask))
  (pad 1 thru_hole circle (at 5.08 17.78) (size 1.524 1.524) (drill 1.016) (layers *.Cu *.Mask))
  (pad 1 thru_hole circle (at 5.08 15.24) (size 1.524 1.524) (drill 1.016) (layers *.Cu *.Mask))
  (pad 1 thru_hole circle (at 5.08 12.7) (size 1.524 1.524) (drill 1.016) (layers *.Cu *.Mask))
  (pad 1 thru_hole circle (at 5.08 10.16) (size 1.524 1.524) (drill 1.016) (layers *.Cu *.Mask))
  (pad 1 thru_hole circle (at 5.08 7.62) (size 1.524 1.524) (drill 1.016) (layers *.Cu *.Mask))
  (pad 1 thru_hole circle (at 2.54 7.62) (size 1.524 1.524) (drill 1.016) (layers *.Cu *.Mask))
  (pad 1 thru_hole circle (at 2.54 17.78) (size 1.524 1.524) (drill 1.016) (layers *.Cu *.Mask))
  (pad 1 thru_hole circle (at 2.54 10.16) (size 1.524 1.524) (drill 1.016) (layers *.Cu *.Mask))
  (pad 1 thru_hole circle (at 2.54 15.24) (size 1.524 1.524) (drill 1.016) (layers *.Cu *.Mask))
  (pad 1 thru_hole circle (at 2.54 12.7) (size 1.524 1.524) (drill 1.016) (layers *.Cu *.Mask))
  (pad 1 thru_hole circle (at 0 17.78) (size 1.524 1.524) (drill 1.016) (layers *.Cu *.Mask))
  (pad 1 thru_hole circle (at 0 15.24) (size 1.524 1.524) (drill 1.016) (layers *.Cu *.Mask))
  (pad 1 thru_hole circle (at 0 12.7) (size 1.524 1.524) (drill 1.016) (layers *.Cu *.Mask))
  (pad 1 thru_hole circle (at 0 10.16) (size 1.524 1.524) (drill 1.016) (layers *.Cu *.Mask))
  (pad 1 thru_hole circle (at 0 7.62) (size 1.524 1.524) (drill 1.016) (layers *.Cu *.Mask)))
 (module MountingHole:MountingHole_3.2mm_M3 (layer F.Cu) (at 194.31 80.01)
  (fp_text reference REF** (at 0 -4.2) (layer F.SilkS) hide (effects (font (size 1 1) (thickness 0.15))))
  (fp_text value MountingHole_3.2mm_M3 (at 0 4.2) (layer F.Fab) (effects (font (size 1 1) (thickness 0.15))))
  (pad 1 np_thru_hole circle (at 0 0) (size 3.2 3.2) (drill 3.2) (layers *.Cu *.Mask)))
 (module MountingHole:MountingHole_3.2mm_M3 (layer F.Cu) (at 229.87 80.01)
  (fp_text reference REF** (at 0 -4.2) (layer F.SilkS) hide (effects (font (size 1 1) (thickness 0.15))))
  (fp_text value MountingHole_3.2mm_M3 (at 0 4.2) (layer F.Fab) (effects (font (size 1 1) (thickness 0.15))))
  (pad 1 np_thru_hole circle (at 0 0) (size 3.2 3.2) (drill 3.2) (layers *.Cu *.Mask)))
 (gr_line (start 187.96 104.14) (end 236.22 104.14) (layer Edge.Cuts) (width 0.05))
 (gr_line (start 187.96 55.88) (end 236.22 55.88) (layer Edge.Cuts) (width 0.05))
 (gr_line (start 187.96 55.88) (end 187.96 104.14) (layer Edge.Cuts) (width 0.05))
 (gr_line (start 236.22 55.88) (end 236.22 104.14) (layer Edge.Cuts) (width 0.1))
 (segment (start 203.2 66.04) (end 203.2 76.2) (width 0.4064) (layer F.Cu) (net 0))
 (segment (start 193.04 66.04) (end 193.04 76.2) (width 0.4064) (layer F.Cu) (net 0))
 (segment (start 200.66 66.04) (end 200.66 76.2) (width 0.4064) (layer F.Cu) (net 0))
 (segment (start 205.74 66.04) (end 205.74 76.2) (width 0.4064) (layer F.Cu) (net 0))
 (segment (start 195.58 66.04) (end 195.58 76.2) (width 0.4064) (layer F.Cu) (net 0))
 (segment (start 208.28 66.04) (end 208.28 76.2) (width 0.4064) (layer F.Cu) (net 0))
 (segment (start 198.12 66.04) (end 198.12 76.2) (width 0.4064) (layer F.Cu) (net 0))
 (segment (start 210.82 66.04) (end 210.82 76.2) (width 0.4064) (layer F.Cu) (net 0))
 (segment (start 215.9 66.04) (end 215.9 76.2) (width 0.4064) (layer F.Cu) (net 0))
 (segment (start 218.44 66.04) (end 218.44 76.2) (width 0.4064) (layer F.Cu) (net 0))
 (segment (start 220.98 66.04) (end 220.98 76.2) (width 0.4064) (layer F.Cu) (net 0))
 (segment (start 228.6 66.04) (end 228.6 76.2) (width 0.4064) (layer F.Cu) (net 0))
 (segment (start 223.52 66.04) (end 223.52 76.2) (width 0.4064) (layer F.Cu) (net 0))
 (segment (start 213.36 66.04) (end 213.36 76.2) (width 0.4064) (layer F.Cu) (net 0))
 (segment (start 231.14 66.04) (end 231.14 76.2) (width 0.4064) (layer F.Cu) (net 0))
 (segment (start 226.06 66.04) (end 226.06 76.2) (width 0.4064) (layer F.Cu) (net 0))
 (segment (start 195.58 83.82) (end 195.58 93.98) (width 0.4064) (layer F.Cu) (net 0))
 (segment (start 213.36 83.82) (end 213.36 93.98) (width 0.4064) (layer F.Cu) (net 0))
 (segment (start 220.98 83.82) (end 220.98 93.98) (width 0.4064) (layer F.Cu) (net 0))
 (segment (start 228.6 83.82) (end 228.6 93.98) (width 0.4064) (layer F.Cu) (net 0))
 (segment (start 198.12 83.82) (end 198.12 93.98) (width 0.4064) (layer F.Cu) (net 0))
 (segment (start 218.44 83.82) (end 218.44 93.98) (width 0.4064) (layer F.Cu) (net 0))
 (segment (start 200.66 83.82) (end 200.66 93.98) (width 0.4064) (layer F.Cu) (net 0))
 (segment (start 208.28 83.82) (end 208.28 93.98) (width 0.4064) (layer F.Cu) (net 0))
 (segment (start 203.2 83.82) (end 203.2 93.98) (width 0.4064) (layer F.Cu) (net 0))
 (segment (start 231.14 83.82) (end 231.14 93.98) (width 0.4064) (layer F.Cu) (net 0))
 (segment (start 226.06 83.82) (end 226.06 93.98) (width 0.4064) (layer F.Cu) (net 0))
 (segment (start 193.04 83.82) (end 193.04 93.98) (width 0.4064) (layer F.Cu) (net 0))
 (segment (start 210.82 83.82) (end 210.82 93.98) (width 0.4064) (layer F.Cu) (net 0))
 (segment (start 205.74 83.82) (end 205.74 93.98) (width 0.4064) (layer F.Cu) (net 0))
 (segment (start 223.52 83.82) (end 223.52 93.98) (width 0.4064) (layer F.Cu) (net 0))
 (segment (start 215.9 83.82) (end 215.9 93.98) (width 0.4064) (layer F.Cu) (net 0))
 (segment (start 193.04 58.42) (end 231.14 58.42) (width 0.4064) (layer F.Cu) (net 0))
 (segment (start 193.04 60.96) (end 231.14 60.96) (width 0.4064) (layer F.Cu) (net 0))
 (segment (start 193.04 99.06) (end 231.14 99.06) (width 0.4064) (layer F.Cu) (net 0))
 (segment (start 193.04 101.6) (end 231.14 101.6) (width 0.4064) (layer F.Cu) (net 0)))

